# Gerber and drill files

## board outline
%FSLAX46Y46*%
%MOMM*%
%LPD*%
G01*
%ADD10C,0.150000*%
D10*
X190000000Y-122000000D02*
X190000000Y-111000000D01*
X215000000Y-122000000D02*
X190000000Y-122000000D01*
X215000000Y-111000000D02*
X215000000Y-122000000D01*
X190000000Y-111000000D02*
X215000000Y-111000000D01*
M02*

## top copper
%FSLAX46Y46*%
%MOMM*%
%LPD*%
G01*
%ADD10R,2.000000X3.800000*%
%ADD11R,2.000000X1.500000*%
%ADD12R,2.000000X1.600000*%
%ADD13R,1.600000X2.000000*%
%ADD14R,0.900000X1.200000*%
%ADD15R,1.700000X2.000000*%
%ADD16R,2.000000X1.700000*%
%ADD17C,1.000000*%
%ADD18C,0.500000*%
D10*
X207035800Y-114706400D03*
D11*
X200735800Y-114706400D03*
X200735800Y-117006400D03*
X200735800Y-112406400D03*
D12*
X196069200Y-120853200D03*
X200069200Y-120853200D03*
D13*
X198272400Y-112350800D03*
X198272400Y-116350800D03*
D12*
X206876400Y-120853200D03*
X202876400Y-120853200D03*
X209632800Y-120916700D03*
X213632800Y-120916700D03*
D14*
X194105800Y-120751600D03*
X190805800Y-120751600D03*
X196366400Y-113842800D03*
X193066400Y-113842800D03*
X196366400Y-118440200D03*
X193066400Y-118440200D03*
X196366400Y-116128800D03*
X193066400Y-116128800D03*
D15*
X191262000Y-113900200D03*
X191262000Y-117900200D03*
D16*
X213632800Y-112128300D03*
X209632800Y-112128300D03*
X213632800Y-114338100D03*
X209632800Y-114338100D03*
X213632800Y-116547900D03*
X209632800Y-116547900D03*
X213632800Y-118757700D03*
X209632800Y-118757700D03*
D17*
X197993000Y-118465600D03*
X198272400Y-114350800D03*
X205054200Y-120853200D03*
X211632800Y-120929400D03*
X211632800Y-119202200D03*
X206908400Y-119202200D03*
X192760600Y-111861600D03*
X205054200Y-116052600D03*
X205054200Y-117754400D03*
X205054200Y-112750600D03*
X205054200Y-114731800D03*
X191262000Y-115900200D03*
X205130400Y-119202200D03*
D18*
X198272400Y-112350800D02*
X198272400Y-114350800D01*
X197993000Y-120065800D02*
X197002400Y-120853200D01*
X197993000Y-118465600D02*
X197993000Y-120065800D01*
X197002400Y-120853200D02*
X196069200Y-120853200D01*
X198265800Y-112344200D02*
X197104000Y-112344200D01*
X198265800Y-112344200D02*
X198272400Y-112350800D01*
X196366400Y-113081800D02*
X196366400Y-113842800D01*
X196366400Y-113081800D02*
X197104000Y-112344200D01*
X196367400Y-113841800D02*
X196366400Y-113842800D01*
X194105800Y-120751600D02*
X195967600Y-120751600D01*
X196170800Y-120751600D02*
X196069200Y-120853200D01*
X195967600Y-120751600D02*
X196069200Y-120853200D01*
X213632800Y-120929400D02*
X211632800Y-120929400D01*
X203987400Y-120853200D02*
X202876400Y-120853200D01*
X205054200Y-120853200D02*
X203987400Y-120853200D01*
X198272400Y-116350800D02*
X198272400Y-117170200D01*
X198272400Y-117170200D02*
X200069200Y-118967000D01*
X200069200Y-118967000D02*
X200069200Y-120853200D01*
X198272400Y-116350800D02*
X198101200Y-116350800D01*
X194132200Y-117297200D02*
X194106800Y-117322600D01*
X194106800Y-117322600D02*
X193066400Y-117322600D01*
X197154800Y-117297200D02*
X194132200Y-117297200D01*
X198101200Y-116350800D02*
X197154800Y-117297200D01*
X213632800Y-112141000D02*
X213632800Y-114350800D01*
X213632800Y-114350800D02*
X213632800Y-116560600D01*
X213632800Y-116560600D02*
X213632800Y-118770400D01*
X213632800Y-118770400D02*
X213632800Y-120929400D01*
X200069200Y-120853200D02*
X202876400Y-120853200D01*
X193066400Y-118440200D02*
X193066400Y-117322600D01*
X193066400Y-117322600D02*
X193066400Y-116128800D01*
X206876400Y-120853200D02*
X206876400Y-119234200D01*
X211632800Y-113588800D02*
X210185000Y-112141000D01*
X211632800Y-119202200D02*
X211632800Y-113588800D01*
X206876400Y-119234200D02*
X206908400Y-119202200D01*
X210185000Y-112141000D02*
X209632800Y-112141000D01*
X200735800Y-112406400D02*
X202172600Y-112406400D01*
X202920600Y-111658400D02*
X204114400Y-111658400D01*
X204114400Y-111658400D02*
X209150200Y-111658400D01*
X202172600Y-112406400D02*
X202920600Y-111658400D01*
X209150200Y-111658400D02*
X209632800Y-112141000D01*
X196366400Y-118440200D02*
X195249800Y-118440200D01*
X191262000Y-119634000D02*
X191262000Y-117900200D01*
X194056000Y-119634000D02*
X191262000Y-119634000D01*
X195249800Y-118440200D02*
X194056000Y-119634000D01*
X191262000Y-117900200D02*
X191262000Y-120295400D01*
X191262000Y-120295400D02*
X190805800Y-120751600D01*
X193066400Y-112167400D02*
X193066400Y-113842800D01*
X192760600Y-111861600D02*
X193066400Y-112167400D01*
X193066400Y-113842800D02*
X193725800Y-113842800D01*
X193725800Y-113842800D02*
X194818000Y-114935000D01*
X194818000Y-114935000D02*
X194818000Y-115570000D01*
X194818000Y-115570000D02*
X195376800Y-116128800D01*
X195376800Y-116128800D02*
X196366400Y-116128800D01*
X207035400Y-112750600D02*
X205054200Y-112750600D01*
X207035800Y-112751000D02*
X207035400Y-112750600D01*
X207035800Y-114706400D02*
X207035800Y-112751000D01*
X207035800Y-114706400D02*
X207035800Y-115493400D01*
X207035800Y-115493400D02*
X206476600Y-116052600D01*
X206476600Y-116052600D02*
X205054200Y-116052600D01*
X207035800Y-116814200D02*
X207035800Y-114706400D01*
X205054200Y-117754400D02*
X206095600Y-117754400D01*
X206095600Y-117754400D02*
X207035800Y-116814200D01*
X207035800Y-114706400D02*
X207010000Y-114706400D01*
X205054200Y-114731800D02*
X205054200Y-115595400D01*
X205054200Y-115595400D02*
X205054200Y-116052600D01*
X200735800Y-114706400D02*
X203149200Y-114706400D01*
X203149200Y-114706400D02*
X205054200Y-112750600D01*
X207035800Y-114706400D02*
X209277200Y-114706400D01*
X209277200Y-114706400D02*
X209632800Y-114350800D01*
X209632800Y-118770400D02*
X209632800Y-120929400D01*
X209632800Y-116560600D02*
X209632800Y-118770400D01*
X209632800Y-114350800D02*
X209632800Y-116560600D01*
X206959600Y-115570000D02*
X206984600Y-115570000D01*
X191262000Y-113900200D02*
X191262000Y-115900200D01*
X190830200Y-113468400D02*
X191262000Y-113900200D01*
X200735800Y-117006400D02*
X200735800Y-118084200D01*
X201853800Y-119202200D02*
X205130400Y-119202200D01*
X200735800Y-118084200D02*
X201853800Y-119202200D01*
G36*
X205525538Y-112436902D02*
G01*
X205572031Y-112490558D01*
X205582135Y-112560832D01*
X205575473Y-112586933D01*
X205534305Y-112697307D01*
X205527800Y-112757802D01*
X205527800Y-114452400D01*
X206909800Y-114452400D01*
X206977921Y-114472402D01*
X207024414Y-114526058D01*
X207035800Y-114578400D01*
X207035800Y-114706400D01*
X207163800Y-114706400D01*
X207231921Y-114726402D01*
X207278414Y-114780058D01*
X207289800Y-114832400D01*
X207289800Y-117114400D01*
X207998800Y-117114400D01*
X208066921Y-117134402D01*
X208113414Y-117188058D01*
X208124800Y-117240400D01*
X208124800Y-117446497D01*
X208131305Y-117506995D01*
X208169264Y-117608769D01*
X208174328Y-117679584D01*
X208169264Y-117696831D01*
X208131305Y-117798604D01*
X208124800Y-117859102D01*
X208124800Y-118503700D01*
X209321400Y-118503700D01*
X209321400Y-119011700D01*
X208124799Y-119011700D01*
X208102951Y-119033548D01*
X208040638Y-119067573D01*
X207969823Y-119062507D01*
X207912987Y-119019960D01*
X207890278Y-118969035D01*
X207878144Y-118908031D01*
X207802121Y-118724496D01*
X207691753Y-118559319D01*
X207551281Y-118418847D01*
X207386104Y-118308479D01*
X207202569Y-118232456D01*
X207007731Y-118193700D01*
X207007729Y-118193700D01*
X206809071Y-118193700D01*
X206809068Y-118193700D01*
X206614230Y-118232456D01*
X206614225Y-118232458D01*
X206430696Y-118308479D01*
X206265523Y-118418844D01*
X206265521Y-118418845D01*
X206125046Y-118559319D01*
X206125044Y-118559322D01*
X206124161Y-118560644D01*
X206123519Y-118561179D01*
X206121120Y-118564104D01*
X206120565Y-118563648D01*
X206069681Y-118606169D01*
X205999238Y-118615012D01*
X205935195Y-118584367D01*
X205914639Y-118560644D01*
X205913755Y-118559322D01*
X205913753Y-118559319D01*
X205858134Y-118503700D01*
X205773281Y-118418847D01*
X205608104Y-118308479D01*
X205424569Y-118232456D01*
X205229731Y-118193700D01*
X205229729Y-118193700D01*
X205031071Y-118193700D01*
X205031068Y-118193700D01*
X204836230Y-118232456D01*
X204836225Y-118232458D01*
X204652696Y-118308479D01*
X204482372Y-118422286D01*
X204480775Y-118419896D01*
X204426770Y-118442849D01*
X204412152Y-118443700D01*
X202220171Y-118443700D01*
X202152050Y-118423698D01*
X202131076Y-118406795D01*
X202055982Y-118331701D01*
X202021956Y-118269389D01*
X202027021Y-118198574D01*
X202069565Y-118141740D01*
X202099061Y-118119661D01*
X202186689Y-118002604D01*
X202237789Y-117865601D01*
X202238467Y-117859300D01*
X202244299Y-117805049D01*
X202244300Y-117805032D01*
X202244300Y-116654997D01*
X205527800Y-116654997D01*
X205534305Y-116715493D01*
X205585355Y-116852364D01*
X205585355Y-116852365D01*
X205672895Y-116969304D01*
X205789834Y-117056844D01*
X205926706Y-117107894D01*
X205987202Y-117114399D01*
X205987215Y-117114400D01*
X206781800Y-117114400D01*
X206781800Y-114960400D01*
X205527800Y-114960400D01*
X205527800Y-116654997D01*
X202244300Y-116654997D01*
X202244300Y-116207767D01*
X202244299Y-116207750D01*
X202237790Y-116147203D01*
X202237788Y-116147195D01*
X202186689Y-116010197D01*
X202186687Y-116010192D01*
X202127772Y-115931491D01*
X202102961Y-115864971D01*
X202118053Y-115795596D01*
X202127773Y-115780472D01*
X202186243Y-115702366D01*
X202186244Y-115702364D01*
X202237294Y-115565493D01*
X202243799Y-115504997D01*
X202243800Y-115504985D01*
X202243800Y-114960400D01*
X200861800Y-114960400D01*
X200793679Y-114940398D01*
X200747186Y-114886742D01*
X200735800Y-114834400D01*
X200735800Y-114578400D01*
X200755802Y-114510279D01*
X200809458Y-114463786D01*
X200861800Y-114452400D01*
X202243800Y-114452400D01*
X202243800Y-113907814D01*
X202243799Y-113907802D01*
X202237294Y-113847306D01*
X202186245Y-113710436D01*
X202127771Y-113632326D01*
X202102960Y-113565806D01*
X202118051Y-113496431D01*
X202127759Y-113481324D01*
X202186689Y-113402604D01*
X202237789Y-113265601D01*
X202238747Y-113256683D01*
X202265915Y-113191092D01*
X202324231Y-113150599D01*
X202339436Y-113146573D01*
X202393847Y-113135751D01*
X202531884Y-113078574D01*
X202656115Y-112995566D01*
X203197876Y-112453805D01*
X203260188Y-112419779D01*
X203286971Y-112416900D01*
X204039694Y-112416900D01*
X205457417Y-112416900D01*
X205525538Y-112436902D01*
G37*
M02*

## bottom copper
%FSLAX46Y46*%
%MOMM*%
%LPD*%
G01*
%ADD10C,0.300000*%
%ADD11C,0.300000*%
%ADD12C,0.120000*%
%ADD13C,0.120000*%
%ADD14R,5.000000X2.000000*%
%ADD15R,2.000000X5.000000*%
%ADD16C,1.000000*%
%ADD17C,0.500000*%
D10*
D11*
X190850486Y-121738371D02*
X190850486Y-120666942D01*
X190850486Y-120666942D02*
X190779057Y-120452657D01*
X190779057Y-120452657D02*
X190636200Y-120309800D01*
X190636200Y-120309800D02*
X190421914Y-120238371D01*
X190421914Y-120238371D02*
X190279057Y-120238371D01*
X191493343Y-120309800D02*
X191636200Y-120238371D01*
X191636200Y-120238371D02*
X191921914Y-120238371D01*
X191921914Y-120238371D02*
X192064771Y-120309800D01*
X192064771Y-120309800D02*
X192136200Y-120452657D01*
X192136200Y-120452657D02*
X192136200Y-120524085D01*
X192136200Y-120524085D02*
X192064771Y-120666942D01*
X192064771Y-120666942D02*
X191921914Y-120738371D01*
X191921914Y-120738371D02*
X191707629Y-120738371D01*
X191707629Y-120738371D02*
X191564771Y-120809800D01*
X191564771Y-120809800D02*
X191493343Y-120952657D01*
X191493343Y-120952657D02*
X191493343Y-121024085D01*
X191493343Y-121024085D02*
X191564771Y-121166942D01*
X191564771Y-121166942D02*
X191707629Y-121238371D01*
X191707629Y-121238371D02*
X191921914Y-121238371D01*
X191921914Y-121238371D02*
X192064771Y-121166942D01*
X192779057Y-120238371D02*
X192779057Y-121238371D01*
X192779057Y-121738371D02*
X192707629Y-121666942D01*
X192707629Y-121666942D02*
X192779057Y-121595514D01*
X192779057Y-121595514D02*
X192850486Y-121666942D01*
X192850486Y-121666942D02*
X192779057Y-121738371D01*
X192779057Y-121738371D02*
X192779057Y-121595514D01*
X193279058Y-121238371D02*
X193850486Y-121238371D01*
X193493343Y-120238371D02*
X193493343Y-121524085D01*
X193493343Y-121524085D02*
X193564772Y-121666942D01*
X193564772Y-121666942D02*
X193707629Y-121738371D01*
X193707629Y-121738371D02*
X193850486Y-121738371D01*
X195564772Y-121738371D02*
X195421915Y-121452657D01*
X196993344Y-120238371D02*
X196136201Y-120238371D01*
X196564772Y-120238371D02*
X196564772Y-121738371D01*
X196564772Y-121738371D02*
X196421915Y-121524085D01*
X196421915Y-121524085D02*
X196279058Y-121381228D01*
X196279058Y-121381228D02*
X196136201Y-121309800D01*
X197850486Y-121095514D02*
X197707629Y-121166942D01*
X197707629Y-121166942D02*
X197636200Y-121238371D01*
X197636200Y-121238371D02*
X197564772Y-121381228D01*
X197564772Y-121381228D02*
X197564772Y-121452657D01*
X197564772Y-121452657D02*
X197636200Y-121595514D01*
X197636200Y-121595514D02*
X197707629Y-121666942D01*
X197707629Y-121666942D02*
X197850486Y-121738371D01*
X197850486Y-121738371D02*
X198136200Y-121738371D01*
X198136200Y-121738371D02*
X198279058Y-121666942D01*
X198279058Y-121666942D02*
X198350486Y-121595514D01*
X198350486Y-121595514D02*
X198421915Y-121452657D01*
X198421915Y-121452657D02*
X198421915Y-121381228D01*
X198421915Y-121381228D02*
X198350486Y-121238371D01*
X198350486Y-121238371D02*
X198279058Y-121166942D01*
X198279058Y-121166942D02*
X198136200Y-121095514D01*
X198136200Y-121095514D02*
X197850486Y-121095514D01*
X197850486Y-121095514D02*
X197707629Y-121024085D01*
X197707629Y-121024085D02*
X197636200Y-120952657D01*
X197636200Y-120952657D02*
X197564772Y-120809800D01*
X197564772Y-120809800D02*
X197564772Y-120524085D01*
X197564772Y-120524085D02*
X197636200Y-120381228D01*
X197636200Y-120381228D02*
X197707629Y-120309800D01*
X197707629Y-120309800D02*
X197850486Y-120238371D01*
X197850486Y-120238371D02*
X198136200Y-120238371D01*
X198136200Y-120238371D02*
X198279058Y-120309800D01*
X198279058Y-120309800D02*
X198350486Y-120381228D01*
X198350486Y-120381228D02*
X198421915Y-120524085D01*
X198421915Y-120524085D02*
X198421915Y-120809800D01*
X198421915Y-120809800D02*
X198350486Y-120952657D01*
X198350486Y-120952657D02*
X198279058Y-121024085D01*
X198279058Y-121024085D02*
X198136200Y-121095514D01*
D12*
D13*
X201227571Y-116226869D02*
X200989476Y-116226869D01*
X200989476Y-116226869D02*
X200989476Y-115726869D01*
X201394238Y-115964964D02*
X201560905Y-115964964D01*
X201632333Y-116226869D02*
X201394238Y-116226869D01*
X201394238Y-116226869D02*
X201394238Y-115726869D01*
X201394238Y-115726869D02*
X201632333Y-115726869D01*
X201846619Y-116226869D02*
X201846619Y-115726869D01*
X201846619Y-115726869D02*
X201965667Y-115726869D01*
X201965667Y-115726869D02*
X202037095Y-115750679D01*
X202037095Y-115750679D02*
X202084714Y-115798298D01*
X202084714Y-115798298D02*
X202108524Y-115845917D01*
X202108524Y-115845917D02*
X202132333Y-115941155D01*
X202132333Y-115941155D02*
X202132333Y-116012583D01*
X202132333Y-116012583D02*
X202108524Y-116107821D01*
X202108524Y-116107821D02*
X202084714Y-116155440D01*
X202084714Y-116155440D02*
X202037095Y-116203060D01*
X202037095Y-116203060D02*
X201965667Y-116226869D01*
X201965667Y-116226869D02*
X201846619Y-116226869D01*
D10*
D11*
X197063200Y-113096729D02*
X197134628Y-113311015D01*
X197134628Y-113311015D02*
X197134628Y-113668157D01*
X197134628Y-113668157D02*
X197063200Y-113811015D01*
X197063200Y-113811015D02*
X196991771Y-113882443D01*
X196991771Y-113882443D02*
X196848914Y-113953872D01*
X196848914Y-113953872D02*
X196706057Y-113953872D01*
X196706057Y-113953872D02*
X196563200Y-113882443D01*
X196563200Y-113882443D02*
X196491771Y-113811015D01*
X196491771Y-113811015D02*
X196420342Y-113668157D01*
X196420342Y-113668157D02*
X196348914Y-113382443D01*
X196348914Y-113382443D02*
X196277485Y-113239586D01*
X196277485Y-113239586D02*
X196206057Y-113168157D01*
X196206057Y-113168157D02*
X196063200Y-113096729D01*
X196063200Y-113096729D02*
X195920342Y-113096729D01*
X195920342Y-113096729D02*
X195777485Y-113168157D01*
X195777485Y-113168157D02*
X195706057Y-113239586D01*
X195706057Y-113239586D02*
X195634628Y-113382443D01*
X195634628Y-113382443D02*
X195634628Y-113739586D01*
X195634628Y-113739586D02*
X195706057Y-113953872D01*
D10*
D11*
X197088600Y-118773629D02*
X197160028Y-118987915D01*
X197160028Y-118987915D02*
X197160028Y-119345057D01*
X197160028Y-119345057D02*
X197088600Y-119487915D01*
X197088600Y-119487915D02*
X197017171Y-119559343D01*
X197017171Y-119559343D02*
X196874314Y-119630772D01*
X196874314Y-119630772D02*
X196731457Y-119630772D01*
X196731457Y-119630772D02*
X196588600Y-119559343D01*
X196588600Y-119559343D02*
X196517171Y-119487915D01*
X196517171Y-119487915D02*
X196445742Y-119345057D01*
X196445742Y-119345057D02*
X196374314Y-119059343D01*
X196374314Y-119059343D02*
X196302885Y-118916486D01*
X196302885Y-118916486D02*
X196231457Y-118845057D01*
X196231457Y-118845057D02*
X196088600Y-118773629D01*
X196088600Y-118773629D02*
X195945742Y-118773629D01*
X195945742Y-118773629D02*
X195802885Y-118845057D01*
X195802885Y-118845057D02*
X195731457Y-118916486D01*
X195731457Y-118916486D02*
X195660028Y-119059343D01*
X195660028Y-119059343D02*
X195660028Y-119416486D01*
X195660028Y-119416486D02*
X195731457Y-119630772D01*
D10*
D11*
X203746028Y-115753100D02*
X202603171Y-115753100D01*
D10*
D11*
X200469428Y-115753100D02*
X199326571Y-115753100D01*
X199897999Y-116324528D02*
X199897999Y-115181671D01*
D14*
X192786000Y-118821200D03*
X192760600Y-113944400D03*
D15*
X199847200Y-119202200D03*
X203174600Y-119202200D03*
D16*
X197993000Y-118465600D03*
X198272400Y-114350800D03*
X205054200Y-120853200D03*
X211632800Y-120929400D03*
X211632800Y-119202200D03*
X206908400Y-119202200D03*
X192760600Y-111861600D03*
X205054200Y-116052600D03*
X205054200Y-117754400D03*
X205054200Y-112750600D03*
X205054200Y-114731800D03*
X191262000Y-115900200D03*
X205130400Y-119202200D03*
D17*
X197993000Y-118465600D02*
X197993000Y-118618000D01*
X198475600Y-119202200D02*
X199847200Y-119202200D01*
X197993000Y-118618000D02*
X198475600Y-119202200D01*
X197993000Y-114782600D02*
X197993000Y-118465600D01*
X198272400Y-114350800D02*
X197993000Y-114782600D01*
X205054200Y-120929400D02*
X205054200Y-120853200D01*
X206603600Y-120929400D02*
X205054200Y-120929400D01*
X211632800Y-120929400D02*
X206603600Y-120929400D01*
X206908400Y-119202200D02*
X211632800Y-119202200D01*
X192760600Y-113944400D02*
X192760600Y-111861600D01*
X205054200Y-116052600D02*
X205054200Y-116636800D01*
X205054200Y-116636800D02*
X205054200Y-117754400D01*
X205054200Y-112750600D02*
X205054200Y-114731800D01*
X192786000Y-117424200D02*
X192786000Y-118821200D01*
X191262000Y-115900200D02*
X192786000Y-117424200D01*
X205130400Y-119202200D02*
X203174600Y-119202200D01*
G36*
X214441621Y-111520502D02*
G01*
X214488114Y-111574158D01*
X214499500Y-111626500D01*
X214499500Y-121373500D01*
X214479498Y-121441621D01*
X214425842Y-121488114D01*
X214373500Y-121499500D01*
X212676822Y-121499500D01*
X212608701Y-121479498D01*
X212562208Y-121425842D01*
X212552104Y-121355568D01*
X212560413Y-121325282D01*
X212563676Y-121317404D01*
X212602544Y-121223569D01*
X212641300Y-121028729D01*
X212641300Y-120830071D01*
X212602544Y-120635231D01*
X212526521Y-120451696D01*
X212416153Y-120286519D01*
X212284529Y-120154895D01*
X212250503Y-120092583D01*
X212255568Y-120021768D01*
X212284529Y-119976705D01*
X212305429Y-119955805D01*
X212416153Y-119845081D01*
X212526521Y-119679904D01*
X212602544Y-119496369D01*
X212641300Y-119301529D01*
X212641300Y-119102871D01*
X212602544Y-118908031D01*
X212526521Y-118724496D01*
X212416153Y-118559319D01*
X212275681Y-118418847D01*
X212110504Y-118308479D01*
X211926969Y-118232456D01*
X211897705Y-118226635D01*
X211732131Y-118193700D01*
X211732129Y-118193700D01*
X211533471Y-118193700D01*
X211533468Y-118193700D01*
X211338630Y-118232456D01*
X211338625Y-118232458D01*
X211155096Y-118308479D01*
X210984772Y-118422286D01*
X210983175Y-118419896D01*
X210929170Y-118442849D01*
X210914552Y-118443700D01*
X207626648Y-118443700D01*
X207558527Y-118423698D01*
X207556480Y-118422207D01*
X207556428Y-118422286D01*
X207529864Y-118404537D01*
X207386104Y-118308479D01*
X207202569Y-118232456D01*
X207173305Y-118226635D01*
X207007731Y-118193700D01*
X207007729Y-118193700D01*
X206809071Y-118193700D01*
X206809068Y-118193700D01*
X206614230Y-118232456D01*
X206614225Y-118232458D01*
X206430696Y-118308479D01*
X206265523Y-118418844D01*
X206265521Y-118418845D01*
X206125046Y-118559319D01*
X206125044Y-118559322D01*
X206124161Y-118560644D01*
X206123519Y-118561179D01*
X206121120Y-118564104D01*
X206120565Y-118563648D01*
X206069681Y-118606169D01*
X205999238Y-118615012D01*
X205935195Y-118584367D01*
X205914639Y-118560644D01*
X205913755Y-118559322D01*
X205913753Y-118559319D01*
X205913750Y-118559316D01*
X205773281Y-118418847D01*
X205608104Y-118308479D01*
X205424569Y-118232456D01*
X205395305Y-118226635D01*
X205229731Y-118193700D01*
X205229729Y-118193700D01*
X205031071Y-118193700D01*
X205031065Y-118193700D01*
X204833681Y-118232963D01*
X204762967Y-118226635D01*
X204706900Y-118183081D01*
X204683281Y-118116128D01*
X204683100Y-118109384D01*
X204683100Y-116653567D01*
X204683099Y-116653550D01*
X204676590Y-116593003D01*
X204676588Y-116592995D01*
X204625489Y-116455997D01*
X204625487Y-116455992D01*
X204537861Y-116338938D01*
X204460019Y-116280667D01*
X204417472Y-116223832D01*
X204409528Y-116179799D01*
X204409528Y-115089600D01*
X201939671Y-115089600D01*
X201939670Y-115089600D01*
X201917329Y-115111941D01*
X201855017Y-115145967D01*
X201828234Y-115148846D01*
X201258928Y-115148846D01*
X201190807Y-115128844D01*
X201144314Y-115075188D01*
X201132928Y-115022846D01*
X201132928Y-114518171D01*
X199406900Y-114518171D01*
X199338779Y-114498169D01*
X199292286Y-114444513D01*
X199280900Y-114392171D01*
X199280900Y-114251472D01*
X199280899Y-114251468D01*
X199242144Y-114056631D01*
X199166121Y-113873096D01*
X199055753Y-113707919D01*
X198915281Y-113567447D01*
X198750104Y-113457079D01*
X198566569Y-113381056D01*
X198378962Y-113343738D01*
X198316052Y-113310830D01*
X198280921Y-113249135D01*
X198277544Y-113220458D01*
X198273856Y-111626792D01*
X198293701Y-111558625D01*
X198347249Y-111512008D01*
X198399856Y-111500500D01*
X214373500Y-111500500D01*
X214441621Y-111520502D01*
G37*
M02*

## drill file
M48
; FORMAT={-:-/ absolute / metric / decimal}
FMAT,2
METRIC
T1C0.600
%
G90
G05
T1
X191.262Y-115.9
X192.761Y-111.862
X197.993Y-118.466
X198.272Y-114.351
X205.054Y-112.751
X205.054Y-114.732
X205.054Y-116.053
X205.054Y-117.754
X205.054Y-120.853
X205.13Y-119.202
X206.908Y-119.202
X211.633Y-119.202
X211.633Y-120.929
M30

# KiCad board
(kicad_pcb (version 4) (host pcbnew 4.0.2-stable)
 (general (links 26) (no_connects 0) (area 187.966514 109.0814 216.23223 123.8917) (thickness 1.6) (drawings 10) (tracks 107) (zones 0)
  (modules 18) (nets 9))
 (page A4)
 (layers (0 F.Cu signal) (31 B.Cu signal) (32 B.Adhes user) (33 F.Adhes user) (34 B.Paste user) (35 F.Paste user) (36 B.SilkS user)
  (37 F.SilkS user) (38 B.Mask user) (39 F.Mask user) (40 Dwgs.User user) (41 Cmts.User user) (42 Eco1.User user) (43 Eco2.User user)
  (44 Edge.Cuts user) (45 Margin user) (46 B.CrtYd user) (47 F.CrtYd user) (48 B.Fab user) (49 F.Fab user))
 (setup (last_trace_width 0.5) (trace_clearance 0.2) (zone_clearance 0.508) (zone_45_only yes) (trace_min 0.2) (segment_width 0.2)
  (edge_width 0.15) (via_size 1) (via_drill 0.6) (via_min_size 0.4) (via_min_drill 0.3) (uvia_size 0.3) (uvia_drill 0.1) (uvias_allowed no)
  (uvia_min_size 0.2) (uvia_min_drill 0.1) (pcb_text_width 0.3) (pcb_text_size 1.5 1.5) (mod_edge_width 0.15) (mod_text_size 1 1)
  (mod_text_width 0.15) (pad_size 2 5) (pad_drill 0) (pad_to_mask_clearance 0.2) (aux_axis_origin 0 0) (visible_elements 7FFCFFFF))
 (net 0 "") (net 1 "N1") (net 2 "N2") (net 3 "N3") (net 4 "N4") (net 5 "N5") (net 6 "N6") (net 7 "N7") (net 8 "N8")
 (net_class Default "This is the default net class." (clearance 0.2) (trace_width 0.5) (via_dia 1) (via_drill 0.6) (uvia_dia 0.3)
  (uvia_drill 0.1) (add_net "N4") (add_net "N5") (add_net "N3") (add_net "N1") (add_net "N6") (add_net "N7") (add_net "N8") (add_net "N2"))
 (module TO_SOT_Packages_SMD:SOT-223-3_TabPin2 (layer F.Cu) (at 203.8858 114.7064)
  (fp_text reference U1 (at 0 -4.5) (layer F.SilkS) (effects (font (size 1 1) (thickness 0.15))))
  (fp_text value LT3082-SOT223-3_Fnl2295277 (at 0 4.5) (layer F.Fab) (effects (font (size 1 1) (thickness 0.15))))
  (pad 2 smd rect (at 3.15 0) (size 2 3.8) (layers F.Cu F.Paste F.Mask) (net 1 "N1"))
  (pad 2 smd rect (at -3.15 0) (size 2 1.5) (layers F.Cu F.Paste F.Mask) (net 1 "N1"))
  (pad 3 smd rect (at -3.15 2.3) (size 2 1.5) (layers F.Cu F.Paste F.Mask) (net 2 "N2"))
  (pad 1 smd rect (at -3.15 -2.3) (size 2 1.5) (layers F.Cu F.Paste F.Mask) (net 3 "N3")))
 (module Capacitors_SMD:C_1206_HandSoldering (layer F.Cu) (at 198.0692 120.8532)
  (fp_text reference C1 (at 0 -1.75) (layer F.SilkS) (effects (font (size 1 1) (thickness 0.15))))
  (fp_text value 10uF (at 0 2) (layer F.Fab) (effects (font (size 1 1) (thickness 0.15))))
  (pad 1 smd rect (at -2 0) (size 2 1.6) (layers F.Cu F.Paste F.Mask) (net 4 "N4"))
  (pad 2 smd rect (at 2 0) (size 2 1.6) (layers F.Cu F.Paste F.Mask) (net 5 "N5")))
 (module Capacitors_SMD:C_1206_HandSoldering (layer F.Cu) (at 198.2724 114.3508 270)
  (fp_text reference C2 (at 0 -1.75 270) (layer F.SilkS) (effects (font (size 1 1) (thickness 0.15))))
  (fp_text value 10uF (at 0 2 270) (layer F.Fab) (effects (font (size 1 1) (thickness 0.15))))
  (pad 1 smd rect (at -2 0 270) (size 2 1.6) (layers F.Cu F.Paste F.Mask) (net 4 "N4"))
  (pad 2 smd rect (at 2 0 270) (size 2 1.6) (layers F.Cu F.Paste F.Mask) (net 5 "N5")))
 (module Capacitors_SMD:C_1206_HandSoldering (layer F.Cu) (at 204.8764 120.8532 180)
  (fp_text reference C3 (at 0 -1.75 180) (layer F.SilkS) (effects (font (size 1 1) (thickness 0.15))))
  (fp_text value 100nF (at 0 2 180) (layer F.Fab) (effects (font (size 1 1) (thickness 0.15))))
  (pad 1 smd rect (at -2 0 180) (size 2 1.6) (layers F.Cu F.Paste F.Mask) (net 3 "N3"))
  (pad 2 smd rect (at 2 0 180) (size 2 1.6) (layers F.Cu F.Paste F.Mask) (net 5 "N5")))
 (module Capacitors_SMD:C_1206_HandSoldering (layer F.Cu) (at 211.6328 120.9167)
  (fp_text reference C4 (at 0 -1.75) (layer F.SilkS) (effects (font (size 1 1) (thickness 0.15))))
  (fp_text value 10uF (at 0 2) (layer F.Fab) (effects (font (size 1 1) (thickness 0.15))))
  (pad 1 smd rect (at -2 0) (size 2 1.6) (layers F.Cu F.Paste F.Mask) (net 1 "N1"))
  (pad 2 smd rect (at 2 0) (size 2 1.6) (layers F.Cu F.Paste F.Mask) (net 5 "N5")))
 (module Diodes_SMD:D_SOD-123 (layer F.Cu) (at 192.4558 120.7516 180)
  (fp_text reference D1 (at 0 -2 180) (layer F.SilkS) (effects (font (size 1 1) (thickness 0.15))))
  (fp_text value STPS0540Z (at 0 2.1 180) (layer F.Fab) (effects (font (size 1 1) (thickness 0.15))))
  (pad 1 smd rect (at -1.65 0 180) (size 0.9 1.2) (layers F.Cu F.Paste F.Mask) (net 4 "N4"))
  (pad 2 smd rect (at 1.65 0 180) (size 0.9 1.2) (layers F.Cu F.Paste F.Mask) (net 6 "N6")))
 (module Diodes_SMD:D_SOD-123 (layer F.Cu) (at 194.7164 113.8428 180)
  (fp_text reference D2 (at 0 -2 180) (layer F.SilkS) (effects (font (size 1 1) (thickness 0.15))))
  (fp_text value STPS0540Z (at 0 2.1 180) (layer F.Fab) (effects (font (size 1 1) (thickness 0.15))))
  (pad 1 smd rect (at -1.65 0 180) (size 0.9 1.2) (layers F.Cu F.Paste F.Mask) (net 4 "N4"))
  (pad 2 smd rect (at 1.65 0 180) (size 0.9 1.2) (layers F.Cu F.Paste F.Mask) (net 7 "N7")))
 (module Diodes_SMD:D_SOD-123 (layer F.Cu) (at 194.7164 118.4402 180)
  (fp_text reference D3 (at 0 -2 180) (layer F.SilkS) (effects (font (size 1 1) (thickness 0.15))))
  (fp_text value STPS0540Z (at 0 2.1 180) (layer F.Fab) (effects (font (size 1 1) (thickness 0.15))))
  (pad 1 smd rect (at -1.65 0 180) (size 0.9 1.2) (layers F.Cu F.Paste F.Mask) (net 6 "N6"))
  (pad 2 smd rect (at 1.65 0 180) (size 0.9 1.2) (layers F.Cu F.Paste F.Mask) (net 5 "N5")))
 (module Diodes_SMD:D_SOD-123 (layer F.Cu) (at 194.7164 116.1288 180)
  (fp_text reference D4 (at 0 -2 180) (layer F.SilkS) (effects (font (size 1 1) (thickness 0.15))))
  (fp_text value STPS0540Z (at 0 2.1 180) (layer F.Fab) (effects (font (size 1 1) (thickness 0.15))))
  (pad 1 smd rect (at -1.65 0 180) (size 0.9 1.2) (layers F.Cu F.Paste F.Mask) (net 7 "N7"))
  (pad 2 smd rect (at 1.65 0 180) (size 0.9 1.2) (layers F.Cu F.Paste F.Mask) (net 5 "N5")))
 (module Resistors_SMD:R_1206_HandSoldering (layer F.Cu) (at 191.262 115.9002 270)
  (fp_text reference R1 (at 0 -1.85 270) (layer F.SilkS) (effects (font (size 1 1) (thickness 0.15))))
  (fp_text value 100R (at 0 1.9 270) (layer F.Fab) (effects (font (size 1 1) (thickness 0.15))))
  (pad 1 smd rect (at -2 0 270) (size 2 1.7) (layers F.Cu F.Paste F.Mask) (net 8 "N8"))
  (pad 2 smd rect (at 2 0 270) (size 2 1.7) (layers F.Cu F.Paste F.Mask) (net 6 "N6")))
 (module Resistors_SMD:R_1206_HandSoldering (layer F.Cu) (at 211.6328 112.1283 180)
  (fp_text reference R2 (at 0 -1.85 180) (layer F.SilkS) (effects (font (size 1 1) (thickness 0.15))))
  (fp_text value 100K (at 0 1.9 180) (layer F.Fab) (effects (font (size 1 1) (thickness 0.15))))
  (pad 1 smd rect (at -2 0 180) (size 2 1.7) (layers F.Cu F.Paste F.Mask) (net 5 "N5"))
  (pad 2 smd rect (at 2 0 180) (size 2 1.7) (layers F.Cu F.Paste F.Mask) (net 3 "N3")))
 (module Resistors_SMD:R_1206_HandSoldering (layer F.Cu) (at 211.6328 114.3381 180)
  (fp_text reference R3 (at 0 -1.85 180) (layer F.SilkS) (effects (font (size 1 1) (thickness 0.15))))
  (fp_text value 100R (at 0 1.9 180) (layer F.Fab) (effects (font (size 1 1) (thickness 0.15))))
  (pad 1 smd rect (at -2 0 180) (size 2 1.7) (layers F.Cu F.Paste F.Mask) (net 5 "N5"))
  (pad 2 smd rect (at 2 0 180) (size 2 1.7) (layers F.Cu F.Paste F.Mask) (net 1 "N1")))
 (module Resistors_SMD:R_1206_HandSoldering (layer F.Cu) (at 211.6328 116.5479 180)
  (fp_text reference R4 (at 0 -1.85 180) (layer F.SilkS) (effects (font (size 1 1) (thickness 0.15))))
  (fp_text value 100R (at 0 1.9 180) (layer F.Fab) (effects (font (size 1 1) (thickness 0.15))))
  (pad 1 smd rect (at -2 0 180) (size 2 1.7) (layers F.Cu F.Paste F.Mask) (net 5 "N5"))
  (pad 2 smd rect (at 2 0 180) (size 2 1.7) (layers F.Cu F.Paste F.Mask) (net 1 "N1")))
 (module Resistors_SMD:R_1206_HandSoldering (layer F.Cu) (at 211.6328 118.7577 180)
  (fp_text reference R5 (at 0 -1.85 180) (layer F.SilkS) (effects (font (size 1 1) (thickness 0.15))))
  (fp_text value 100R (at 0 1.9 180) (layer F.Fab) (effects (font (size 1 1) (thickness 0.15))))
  (pad 1 smd rect (at -2 0 180) (size 2 1.7) (layers F.Cu F.Paste F.Mask) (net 5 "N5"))
  (pad 2 smd rect (at 2 0 180) (size 2 1.7) (layers F.Cu F.Paste F.Mask) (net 1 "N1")))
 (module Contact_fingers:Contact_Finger (layer F.Cu) (at 192.786 118.8212 90)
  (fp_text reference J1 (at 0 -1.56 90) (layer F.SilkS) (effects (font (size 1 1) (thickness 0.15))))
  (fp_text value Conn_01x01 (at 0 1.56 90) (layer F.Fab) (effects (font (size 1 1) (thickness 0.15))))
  (pad 1 smd rect (at 0 0 90) (size 2 5) (layers B.Cu B.Paste B.Mask) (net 8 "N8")))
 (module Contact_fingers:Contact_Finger (layer F.Cu) (at 192.7606 113.9444 90)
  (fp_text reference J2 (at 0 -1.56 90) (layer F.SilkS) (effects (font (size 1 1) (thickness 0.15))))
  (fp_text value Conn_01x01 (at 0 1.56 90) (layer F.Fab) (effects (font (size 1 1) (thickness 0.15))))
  (pad 1 smd rect (at 0 0 90) (size 2 5) (layers B.Cu B.Paste B.Mask) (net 7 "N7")))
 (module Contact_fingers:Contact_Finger (layer F.Cu) (at 199.8472 119.2022 180)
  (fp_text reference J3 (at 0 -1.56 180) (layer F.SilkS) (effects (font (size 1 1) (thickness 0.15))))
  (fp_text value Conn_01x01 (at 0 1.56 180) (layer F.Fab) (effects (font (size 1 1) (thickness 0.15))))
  (pad 1 smd rect (at 0 0 180) (size 2 5) (layers B.Cu B.Paste B.Mask) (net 4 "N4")))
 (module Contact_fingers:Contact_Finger (layer F.Cu) (at 203.1746 119.2022 180)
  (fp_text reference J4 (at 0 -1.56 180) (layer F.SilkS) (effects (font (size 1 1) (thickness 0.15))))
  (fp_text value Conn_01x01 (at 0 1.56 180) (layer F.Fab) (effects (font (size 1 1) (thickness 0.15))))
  (pad 1 smd rect (at 0 0 180) (size 2 5) (layers B.Cu B.Paste B.Mask) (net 2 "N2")))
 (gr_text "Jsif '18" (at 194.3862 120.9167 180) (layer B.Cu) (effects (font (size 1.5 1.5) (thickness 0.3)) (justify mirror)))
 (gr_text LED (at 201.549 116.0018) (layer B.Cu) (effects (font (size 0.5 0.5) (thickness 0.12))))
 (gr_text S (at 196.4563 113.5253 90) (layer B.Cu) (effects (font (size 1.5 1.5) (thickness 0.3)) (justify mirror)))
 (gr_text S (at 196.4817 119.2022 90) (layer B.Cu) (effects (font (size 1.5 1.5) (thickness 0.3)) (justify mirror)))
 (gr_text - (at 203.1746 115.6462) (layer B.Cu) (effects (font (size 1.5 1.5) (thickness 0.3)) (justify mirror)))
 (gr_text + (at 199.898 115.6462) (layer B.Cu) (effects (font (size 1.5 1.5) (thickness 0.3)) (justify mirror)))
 (gr_line (start 190 122) (end 190 111) (angle 90) (layer Edge.Cuts) (width 0.15))
 (gr_line (start 215 122) (end 190 122) (angle 90) (layer Edge.Cuts) (width 0.15))
 (gr_line (start 215 111) (end 215 122) (angle 90) (layer Edge.Cuts) (width 0.15))
 (gr_line (start 190 111) (end 215 111) (angle 90) (layer Edge.Cuts) (width 0.15))
 (segment (start 197.993 118.4656) (end 197.993 118.618) (width 0.5) (layer B.Cu) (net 4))
 (segment (start 198.4756 119.2022) (end 199.8472 119.2022) (width 0.5) (layer B.Cu) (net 4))
 (segment (start 197.993 118.618) (end 198.4756 119.2022) (width 0.5) (layer B.Cu) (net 4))
 (segment (start 198.2724 112.3508) (end 198.2724 114.3508) (width 0.5) (layer F.Cu) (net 4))
 (segment (start 197.993 120.0658) (end 197.0024 120.8532) (width 0.5) (layer F.Cu) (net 4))
 (segment (start 197.993 118.4656) (end 197.993 120.0658) (width 0.5) (layer F.Cu) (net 4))
 (via (at 197.993 118.4656) (size 1) (drill 0.6) (layers F.Cu B.Cu) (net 4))
 (segment (start 197.993 114.7826) (end 197.993 118.4656) (width 0.5) (layer B.Cu) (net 4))
 (segment (start 198.2724 114.3508) (end 197.993 114.7826) (width 0.5) (layer B.Cu) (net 4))
 (via (at 198.2724 114.3508) (size 1) (drill 0.6) (layers F.Cu B.Cu) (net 4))
 (segment (start 197.0024 120.8532) (end 196.0692 120.8532) (width 0.5) (layer F.Cu) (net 4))
 (segment (start 198.2658 112.3442) (end 197.104 112.3442) (width 0.5) (layer F.Cu) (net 4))
 (segment (start 198.2658 112.3442) (end 198.2724 112.3508) (width 0.5) (layer F.Cu) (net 4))
 (segment (start 196.3664 113.0818) (end 196.3664 113.8428) (width 0.5) (layer F.Cu) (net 4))
 (segment (start 196.3664 113.0818) (end 197.104 112.3442) (width 0.5) (layer F.Cu) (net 4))
 (segment (start 196.3674 113.8418) (end 196.3664 113.8428) (width 0.5) (layer F.Cu) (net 4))
 (segment (start 194.1058 120.7516) (end 195.9676 120.7516) (width 0.5) (layer F.Cu) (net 4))
 (segment (start 196.1708 120.7516) (end 196.0692 120.8532) (width 0.5) (layer F.Cu) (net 4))
 (segment (start 195.9676 120.7516) (end 196.0692 120.8532) (width 0.5) (layer F.Cu) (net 4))
 (segment (start 213.6328 120.9294) (end 211.6328 120.9294) (width 0.5) (layer F.Cu) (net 5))
 (segment (start 203.9874 120.8532) (end 202.8764 120.8532) (width 0.5) (layer F.Cu) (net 5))
 (segment (start 205.0542 120.8532) (end 203.9874 120.8532) (width 0.5) (layer F.Cu) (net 5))
 (via (at 205.0542 120.8532) (size 1) (drill 0.6) (layers F.Cu B.Cu) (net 5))
 (segment (start 205.0542 120.9294) (end 205.0542 120.8532) (width 0.5) (layer B.Cu) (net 5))
 (segment (start 206.6036 120.9294) (end 205.0542 120.9294) (width 0.5) (layer B.Cu) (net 5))
 (segment (start 211.6328 120.9294) (end 206.6036 120.9294) (width 0.5) (layer B.Cu) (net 5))
 (via (at 211.6328 120.9294) (size 1) (drill 0.6) (layers F.Cu B.Cu) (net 5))
 (segment (start 198.2724 116.3508) (end 198.2724 117.1702) (width 0.5) (layer F.Cu) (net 5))
 (segment (start 198.2724 117.1702) (end 200.0692 118.967) (width 0.5) (layer F.Cu) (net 5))
 (segment (start 200.0692 118.967) (end 200.0692 120.8532) (width 0.5) (layer F.Cu) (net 5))
 (segment (start 198.2724 116.3508) (end 198.1012 116.3508) (width 0.5) (layer F.Cu) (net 5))
 (segment (start 194.1322 117.2972) (end 194.1068 117.3226) (width 0.5) (layer F.Cu) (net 5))
 (segment (start 194.1068 117.3226) (end 193.0664 117.3226) (width 0.5) (layer F.Cu) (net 5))
 (segment (start 197.1548 117.2972) (end 194.1322 117.2972) (width 0.5) (layer F.Cu) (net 5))
 (segment (start 198.1012 116.3508) (end 197.1548 117.2972) (width 0.5) (layer F.Cu) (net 5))
 (segment (start 213.6328 112.141) (end 213.6328 114.3508) (width 0.5) (layer F.Cu) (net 5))
 (segment (start 213.6328 114.3508) (end 213.6328 116.5606) (width 0.5) (layer F.Cu) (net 5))
 (segment (start 213.6328 116.5606) (end 213.6328 118.7704) (width 0.5) (layer F.Cu) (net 5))
 (segment (start 213.6328 118.7704) (end 213.6328 120.9294) (width 0.5) (layer F.Cu) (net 5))
 (segment (start 200.0692 120.8532) (end 202.8764 120.8532) (width 0.5) (layer F.Cu) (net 5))
 (segment (start 193.0664 118.4402) (end 193.0664 117.3226) (width 0.5) (layer F.Cu) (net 5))
 (segment (start 193.0664 117.3226) (end 193.0664 116.1288) (width 0.5) (layer F.Cu) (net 5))
 (segment (start 206.8764 120.8532) (end 206.8764 119.2342) (width 0.5) (layer F.Cu) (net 3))
 (segment (start 211.6328 113.5888) (end 210.185 112.141) (width 0.5) (layer F.Cu) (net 3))
 (segment (start 211.6328 119.2022) (end 211.6328 113.5888) (width 0.5) (layer F.Cu) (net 3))
 (via (at 211.6328 119.2022) (size 1) (drill 0.6) (layers F.Cu B.Cu) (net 3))
 (segment (start 206.9084 119.2022) (end 211.6328 119.2022) (width 0.5) (layer B.Cu) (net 3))
 (via (at 206.9084 119.2022) (size 1) (drill 0.6) (layers F.Cu B.Cu) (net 3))
 (segment (start 206.8764 119.2342) (end 206.9084 119.2022) (width 0.5) (layer F.Cu) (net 3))
 (segment (start 210.185 112.141) (end 209.6328 112.141) (width 0.5) (layer F.Cu) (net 3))
 (segment (start 200.7358 112.4064) (end 202.1726 112.4064) (width 0.5) (layer F.Cu) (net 3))
 (segment (start 202.9206 111.6584) (end 204.1144 111.6584) (width 0.5) (layer F.Cu) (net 3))
 (segment (start 204.1144 111.6584) (end 209.1502 111.6584) (width 0.5) (layer F.Cu) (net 3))
 (segment (start 202.1726 112.4064) (end 202.9206 111.6584) (width 0.5) (layer F.Cu) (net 3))
 (segment (start 209.1502 111.6584) (end 209.6328 112.141) (width 0.5) (layer F.Cu) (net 3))
 (segment (start 196.3664 118.4402) (end 195.2498 118.4402) (width 0.5) (layer F.Cu) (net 6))
 (segment (start 191.262 119.634) (end 191.262 117.9002) (width 0.5) (layer F.Cu) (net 6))
 (segment (start 194.056 119.634) (end 191.262 119.634) (width 0.5) (layer F.Cu) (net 6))
 (segment (start 195.2498 118.4402) (end 194.056 119.634) (width 0.5) (layer F.Cu) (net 6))
 (segment (start 191.262 117.9002) (end 191.262 120.2954) (width 0.5) (layer F.Cu) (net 6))
 (segment (start 191.262 120.2954) (end 190.8058 120.7516) (width 0.5) (layer F.Cu) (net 6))
 (segment (start 192.7606 113.9444) (end 192.7606 111.8616) (width 0.5) (layer B.Cu) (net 7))
 (segment (start 193.0664 112.1674) (end 193.0664 113.8428) (width 0.5) (layer F.Cu) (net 7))
 (segment (start 192.7606 111.8616) (end 193.0664 112.1674) (width 0.5) (layer F.Cu) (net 7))
 (via (at 192.7606 111.8616) (size 1) (drill 0.6) (layers F.Cu B.Cu) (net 7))
 (segment (start 193.0664 113.8428) (end 193.7258 113.8428) (width 0.5) (layer F.Cu) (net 7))
 (segment (start 193.7258 113.8428) (end 194.818 114.935) (width 0.5) (layer F.Cu) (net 7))
 (segment (start 194.818 114.935) (end 194.818 115.57) (width 0.5) (layer F.Cu) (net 7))
 (segment (start 194.818 115.57) (end 195.3768 116.1288) (width 0.5) (layer F.Cu) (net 7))
 (segment (start 195.3768 116.1288) (end 196.3664 116.1288) (width 0.5) (layer F.Cu) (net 7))
 (segment (start 207.0354 112.7506) (end 205.0542 112.7506) (width 0.5) (layer F.Cu) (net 1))
 (segment (start 207.0358 112.751) (end 207.0354 112.7506) (width 0.5) (layer F.Cu) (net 1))
 (segment (start 207.0358 114.7064) (end 207.0358 112.751) (width 0.5) (layer F.Cu) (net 1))
 (segment (start 207.0358 114.7064) (end 207.0358 115.4934) (width 0.5) (layer F.Cu) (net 1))
 (segment (start 207.0358 115.4934) (end 206.4766 116.0526) (width 0.5) (layer F.Cu) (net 1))
 (segment (start 206.4766 116.0526) (end 205.0542 116.0526) (width 0.5) (layer F.Cu) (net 1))
 (segment (start 207.0358 116.8142) (end 207.0358 114.7064) (width 0.5) (layer F.Cu) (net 1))
 (via (at 205.0542 116.0526) (size 1) (drill 0.6) (layers F.Cu B.Cu) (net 1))
 (segment (start 205.0542 116.0526) (end 205.0542 116.6368) (width 0.5) (layer B.Cu) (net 1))
 (segment (start 205.0542 116.6368) (end 205.0542 117.7544) (width 0.5) (layer B.Cu) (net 1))
 (via (at 205.0542 117.7544) (size 1) (drill 0.6) (layers F.Cu B.Cu) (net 1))
 (segment (start 205.0542 117.7544) (end 206.0956 117.7544) (width 0.5) (layer F.Cu) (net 1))
 (segment (start 206.0956 117.7544) (end 207.0358 116.8142) (width 0.5) (layer F.Cu) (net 1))
 (segment (start 207.0358 114.7064) (end 207.01 114.7064) (width 0.5) (layer F.Cu) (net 1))
 (via (at 205.0542 112.7506) (size 1) (drill 0.6) (layers F.Cu B.Cu) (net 1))
 (segment (start 205.0542 112.7506) (end 205.0542 114.7318) (width 0.5) (layer B.Cu) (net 1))
 (via (at 205.0542 114.7318) (size 1) (drill 0.6) (layers F.Cu B.Cu) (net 1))
 (segment (start 205.0542 114.7318) (end 205.0542 115.5954) (width 0.5) (layer F.Cu) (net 1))
 (segment (start 205.0542 115.5954) (end 205.0542 116.0526) (width 0.5) (layer F.Cu) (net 1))
 (segment (start 200.7358 114.7064) (end 203.1492 114.7064) (width 0.5) (layer F.Cu) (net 1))
 (segment (start 203.1492 114.7064) (end 205.0542 112.7506) (width 0.5) (layer F.Cu) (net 1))
 (segment (start 207.0358 114.7064) (end 209.2772 114.7064) (width 0.5) (layer F.Cu) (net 1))
 (segment (start 209.2772 114.7064) (end 209.6328 114.3508) (width 0.5) (layer F.Cu) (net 1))
 (segment (start 209.6328 118.7704) (end 209.6328 120.9294) (width 0.5) (layer F.Cu) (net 1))
 (segment (start 209.6328 116.5606) (end 209.6328 118.7704) (width 0.5) (layer F.Cu) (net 1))
 (segment (start 209.6328 114.3508) (end 209.6328 116.5606) (width 0.5) (layer F.Cu) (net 1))
 (segment (start 206.9596 115.57) (end 206.9846 115.57) (width 0.5) (layer F.Cu) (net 1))
 (segment (start 191.262 113.9002) (end 191.262 115.9002) (width 0.5) (layer F.Cu) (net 8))
 (segment (start 192.786 117.4242) (end 192.786 118.8212) (width 0.5) (layer B.Cu) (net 8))
 (segment (start 191.262 115.9002) (end 192.786 117.4242) (width 0.5) (layer B.Cu) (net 8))
 (via (at 191.262 115.9002) (size 1) (drill 0.6) (layers F.Cu B.Cu) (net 8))
 (segment (start 190.8302 113.4684) (end 191.262 113.9002) (width 0.5) (layer F.Cu) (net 8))
 (segment (start 200.7358 117.0064) (end 200.7358 118.0842) (width 0.5) (layer F.Cu) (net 2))
 (segment (start 205.1304 119.2022) (end 203.1746 119.2022) (width 0.5) (layer B.Cu) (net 2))
 (via (at 205.1304 119.2022) (size 1) (drill 0.6) (layers F.Cu B.Cu) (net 2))
 (segment (start 201.8538 119.2022) (end 205.1304 119.2022) (width 0.5) (layer F.Cu) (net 2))
 (segment (start 200.7358 118.0842) (end 201.8538 119.2022) (width 0.5) (layer F.Cu) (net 2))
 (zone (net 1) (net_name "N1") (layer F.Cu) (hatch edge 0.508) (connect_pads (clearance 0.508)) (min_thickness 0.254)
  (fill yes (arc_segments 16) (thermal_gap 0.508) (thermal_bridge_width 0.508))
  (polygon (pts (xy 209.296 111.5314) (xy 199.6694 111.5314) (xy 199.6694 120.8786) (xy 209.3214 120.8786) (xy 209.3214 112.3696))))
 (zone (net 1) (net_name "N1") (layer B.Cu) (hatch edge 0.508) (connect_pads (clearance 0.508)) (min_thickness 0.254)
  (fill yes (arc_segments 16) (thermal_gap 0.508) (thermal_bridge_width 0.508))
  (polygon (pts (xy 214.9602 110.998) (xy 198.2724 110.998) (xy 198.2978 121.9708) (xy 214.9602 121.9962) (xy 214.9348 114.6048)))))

